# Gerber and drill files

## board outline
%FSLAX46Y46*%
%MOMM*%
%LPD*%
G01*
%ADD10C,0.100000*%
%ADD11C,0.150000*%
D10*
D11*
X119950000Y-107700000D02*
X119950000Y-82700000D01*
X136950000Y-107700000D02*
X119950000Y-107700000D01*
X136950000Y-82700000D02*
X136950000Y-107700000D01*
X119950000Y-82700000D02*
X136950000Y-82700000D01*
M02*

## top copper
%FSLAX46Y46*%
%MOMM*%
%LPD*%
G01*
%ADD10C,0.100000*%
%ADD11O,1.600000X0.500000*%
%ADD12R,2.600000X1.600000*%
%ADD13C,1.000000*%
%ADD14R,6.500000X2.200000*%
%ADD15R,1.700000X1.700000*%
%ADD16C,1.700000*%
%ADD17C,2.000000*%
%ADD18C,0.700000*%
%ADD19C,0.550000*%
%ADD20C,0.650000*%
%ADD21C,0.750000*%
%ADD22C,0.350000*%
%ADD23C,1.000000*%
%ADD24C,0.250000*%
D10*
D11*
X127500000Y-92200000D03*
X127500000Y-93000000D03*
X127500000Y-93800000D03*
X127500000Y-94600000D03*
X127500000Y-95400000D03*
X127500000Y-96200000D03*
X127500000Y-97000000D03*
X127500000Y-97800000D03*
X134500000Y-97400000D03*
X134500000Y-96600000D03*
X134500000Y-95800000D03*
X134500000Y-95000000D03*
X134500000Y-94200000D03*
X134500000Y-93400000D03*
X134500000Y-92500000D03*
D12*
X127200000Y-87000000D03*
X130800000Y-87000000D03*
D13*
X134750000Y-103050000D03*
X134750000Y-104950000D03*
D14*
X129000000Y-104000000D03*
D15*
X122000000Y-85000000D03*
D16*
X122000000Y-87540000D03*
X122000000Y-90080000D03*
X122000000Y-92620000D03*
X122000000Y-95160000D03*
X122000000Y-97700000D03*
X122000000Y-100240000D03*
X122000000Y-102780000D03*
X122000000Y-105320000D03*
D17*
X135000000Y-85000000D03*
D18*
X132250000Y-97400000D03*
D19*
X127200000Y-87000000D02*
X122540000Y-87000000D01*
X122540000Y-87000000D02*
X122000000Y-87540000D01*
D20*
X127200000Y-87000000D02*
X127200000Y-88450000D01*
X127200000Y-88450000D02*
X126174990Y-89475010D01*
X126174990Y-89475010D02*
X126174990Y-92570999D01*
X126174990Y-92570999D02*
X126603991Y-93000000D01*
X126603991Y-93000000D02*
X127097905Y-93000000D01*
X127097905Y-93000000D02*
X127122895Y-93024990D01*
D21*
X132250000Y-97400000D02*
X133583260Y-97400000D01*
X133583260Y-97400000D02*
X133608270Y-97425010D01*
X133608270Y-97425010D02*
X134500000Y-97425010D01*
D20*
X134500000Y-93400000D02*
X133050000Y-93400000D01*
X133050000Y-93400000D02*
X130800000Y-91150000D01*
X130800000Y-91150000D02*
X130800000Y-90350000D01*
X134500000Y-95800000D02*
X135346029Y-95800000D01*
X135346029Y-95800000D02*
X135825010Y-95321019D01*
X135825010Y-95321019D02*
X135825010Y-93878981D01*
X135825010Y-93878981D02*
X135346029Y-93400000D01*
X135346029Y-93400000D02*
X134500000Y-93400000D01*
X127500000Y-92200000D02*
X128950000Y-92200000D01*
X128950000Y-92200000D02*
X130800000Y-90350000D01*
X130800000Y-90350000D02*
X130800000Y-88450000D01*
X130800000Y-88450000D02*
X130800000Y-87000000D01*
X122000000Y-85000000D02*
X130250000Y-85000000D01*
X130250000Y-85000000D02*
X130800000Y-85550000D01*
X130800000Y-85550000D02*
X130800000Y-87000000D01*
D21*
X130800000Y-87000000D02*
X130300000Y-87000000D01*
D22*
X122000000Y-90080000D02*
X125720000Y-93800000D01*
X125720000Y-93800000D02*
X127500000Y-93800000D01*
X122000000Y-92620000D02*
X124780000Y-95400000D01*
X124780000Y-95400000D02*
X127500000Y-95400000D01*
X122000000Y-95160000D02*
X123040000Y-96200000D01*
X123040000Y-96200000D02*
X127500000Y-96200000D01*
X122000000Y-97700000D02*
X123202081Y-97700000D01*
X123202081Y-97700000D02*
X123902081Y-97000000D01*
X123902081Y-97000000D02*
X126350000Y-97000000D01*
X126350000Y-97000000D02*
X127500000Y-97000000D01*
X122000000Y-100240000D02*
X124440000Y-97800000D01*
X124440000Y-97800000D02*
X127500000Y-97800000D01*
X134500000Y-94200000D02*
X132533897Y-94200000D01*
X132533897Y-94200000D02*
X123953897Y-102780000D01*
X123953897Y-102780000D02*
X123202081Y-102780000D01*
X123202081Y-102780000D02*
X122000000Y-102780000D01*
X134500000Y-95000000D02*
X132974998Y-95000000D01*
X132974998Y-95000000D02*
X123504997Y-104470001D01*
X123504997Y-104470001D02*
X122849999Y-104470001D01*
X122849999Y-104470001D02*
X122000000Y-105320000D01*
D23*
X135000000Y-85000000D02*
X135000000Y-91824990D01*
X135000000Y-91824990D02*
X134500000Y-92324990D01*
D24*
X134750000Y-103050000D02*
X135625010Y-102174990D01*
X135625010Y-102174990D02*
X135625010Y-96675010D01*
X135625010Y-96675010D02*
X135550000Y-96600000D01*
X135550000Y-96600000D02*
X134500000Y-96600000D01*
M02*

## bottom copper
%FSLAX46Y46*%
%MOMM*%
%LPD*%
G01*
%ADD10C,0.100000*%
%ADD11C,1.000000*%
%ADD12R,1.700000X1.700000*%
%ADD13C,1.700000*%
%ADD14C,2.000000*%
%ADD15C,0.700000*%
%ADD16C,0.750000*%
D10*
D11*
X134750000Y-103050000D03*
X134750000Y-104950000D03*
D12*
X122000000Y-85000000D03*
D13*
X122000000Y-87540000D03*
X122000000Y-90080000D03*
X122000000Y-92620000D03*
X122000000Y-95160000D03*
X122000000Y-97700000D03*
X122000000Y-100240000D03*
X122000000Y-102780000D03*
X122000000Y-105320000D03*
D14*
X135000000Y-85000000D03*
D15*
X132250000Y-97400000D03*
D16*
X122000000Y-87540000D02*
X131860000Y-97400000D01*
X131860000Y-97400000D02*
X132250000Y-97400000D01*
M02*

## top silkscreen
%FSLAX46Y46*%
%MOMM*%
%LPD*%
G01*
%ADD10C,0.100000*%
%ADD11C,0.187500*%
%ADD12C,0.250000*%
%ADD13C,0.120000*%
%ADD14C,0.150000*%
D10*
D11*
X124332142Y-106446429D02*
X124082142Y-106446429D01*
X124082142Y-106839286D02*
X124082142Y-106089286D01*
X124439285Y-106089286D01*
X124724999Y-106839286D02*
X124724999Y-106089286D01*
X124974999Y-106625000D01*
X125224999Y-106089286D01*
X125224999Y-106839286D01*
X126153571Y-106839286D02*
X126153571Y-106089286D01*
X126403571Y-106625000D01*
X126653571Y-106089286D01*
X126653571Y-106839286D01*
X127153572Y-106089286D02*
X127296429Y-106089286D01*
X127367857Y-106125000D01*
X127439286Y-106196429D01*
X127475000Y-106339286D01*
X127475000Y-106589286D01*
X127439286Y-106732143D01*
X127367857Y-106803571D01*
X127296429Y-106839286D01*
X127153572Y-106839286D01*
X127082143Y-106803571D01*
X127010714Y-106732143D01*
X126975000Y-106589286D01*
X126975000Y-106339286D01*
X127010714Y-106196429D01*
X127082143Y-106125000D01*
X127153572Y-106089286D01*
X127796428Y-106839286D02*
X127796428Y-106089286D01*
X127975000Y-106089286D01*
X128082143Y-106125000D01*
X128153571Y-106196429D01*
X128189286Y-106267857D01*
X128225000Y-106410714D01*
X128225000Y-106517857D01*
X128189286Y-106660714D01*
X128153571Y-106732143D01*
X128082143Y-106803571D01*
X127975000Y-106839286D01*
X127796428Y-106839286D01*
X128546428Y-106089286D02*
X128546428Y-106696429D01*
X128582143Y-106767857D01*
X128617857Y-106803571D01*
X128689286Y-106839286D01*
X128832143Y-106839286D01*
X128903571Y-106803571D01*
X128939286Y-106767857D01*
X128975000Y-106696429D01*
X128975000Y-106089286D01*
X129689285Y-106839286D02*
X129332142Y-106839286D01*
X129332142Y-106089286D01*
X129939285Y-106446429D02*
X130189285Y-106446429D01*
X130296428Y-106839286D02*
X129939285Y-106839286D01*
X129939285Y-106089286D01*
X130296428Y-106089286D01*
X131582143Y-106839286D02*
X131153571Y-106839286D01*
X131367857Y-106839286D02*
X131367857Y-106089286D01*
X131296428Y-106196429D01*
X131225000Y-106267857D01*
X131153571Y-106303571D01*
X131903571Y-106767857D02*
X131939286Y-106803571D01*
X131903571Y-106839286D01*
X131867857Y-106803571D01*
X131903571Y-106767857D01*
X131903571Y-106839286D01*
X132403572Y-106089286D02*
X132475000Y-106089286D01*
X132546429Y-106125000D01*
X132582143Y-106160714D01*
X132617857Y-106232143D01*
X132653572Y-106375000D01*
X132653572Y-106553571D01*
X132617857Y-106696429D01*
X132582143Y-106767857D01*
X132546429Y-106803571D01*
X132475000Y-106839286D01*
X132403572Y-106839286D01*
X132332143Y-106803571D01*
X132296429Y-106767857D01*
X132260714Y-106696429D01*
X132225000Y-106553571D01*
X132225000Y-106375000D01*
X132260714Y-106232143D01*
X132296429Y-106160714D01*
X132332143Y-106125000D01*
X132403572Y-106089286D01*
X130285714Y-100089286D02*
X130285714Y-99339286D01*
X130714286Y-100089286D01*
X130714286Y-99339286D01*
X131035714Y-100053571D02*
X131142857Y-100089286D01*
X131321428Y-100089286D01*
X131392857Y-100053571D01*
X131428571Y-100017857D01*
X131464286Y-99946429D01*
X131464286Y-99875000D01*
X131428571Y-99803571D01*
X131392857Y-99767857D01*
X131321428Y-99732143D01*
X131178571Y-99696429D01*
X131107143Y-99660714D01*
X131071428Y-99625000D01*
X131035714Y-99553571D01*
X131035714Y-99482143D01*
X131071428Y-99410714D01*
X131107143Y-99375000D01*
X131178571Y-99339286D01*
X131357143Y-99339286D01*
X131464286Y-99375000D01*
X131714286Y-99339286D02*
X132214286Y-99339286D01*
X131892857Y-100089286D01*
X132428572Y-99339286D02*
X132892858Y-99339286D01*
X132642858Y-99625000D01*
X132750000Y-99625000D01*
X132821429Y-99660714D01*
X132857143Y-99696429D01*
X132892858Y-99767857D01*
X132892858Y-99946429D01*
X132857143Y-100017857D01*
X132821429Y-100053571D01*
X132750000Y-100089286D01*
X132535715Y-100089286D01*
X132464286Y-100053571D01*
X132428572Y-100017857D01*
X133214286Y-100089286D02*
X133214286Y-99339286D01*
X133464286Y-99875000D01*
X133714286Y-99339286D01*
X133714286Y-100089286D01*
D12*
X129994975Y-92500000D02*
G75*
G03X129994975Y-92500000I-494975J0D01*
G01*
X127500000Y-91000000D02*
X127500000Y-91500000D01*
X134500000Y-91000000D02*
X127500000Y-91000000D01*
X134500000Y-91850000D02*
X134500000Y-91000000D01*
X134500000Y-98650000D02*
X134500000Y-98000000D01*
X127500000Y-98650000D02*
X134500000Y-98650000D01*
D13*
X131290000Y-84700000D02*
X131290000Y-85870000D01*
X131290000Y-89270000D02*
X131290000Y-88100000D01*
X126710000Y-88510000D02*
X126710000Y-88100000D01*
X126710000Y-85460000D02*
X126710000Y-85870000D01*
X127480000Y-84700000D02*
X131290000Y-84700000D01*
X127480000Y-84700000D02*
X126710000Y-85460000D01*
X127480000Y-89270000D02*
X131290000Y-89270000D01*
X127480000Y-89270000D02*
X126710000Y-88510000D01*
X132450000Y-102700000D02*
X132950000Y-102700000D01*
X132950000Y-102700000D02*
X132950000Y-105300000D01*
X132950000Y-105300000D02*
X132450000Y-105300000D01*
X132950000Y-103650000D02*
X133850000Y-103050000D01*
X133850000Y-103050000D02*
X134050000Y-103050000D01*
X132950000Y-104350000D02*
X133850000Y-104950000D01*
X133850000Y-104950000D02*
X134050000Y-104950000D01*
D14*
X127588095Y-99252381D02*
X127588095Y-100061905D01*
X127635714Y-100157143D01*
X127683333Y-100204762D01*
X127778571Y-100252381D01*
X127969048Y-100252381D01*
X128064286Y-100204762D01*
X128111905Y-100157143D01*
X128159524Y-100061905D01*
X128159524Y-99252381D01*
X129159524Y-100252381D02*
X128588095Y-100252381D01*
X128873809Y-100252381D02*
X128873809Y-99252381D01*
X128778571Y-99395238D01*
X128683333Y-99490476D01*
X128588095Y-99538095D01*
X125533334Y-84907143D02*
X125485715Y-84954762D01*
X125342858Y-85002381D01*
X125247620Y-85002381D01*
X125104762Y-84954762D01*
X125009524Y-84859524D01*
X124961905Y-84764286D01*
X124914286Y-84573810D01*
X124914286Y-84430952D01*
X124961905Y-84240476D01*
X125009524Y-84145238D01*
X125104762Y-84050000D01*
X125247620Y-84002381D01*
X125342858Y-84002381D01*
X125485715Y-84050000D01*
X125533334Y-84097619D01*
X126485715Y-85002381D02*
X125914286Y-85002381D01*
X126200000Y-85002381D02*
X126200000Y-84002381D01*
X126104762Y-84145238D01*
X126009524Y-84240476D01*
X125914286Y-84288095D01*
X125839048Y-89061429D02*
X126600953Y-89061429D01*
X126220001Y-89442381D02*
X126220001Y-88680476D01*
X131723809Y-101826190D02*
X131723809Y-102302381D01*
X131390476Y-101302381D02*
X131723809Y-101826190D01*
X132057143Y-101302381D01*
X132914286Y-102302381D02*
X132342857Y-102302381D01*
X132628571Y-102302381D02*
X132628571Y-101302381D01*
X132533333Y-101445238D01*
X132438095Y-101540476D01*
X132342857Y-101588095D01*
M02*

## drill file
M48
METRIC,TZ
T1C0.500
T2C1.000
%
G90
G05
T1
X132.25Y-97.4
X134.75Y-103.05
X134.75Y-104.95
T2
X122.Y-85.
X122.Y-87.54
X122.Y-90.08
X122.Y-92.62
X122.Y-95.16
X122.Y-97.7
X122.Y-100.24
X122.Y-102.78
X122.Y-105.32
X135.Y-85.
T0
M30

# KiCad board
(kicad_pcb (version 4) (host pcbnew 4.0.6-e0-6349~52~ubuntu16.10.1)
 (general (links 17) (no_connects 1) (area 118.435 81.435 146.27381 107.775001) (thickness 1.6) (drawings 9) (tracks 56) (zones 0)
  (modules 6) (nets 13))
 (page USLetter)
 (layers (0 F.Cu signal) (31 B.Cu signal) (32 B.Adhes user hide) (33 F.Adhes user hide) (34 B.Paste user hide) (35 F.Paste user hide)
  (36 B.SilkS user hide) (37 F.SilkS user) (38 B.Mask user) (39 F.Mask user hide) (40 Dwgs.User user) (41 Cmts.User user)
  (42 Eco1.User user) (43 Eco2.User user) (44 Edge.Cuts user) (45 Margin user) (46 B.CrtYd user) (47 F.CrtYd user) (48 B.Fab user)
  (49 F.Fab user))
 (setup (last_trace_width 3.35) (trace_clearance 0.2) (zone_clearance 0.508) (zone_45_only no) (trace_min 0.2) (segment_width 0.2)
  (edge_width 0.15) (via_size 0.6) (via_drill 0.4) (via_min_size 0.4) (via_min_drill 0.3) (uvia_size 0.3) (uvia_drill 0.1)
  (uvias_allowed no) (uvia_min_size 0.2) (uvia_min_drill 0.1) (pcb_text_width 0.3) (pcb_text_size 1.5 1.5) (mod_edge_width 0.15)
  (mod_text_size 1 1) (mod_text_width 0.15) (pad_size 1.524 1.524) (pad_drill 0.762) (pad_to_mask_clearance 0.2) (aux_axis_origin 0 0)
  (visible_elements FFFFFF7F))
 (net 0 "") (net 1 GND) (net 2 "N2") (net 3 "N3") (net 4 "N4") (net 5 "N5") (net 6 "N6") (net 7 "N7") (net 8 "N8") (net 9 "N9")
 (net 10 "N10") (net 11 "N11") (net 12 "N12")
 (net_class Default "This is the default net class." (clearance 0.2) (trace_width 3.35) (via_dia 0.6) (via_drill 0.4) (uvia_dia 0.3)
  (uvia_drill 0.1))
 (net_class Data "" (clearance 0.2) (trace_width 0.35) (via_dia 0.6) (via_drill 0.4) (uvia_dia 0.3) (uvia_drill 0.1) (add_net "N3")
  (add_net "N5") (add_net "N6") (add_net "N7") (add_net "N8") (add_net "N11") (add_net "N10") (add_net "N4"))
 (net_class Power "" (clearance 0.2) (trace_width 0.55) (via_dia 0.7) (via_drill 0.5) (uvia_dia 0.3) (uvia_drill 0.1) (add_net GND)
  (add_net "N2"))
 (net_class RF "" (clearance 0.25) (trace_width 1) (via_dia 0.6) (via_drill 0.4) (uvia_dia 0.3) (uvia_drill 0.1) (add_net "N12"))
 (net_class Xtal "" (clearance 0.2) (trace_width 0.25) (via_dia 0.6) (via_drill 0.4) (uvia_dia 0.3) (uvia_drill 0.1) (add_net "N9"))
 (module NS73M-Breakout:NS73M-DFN (layer F.Cu) (at 131 95 180)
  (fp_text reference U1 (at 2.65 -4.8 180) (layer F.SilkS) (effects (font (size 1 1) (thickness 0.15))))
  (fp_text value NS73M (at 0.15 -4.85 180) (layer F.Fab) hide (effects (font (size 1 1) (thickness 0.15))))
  (fp_circle (center 1.5 2.5) (end 1.15 2.15) (layer F.SilkS) (width 0.25))
  (fp_line (start 3.5 4) (end 3.5 3.5) (layer F.SilkS) (width 0.25))
  (fp_line (start -3.5 4) (end 3.5 4) (layer F.SilkS) (width 0.25))
  (fp_line (start -3.5 3.15) (end -3.5 4) (layer F.SilkS) (width 0.25))
  (fp_line (start -3.5 -3.65) (end -3.5 -3) (layer F.SilkS) (width 0.25))
  (fp_line (start 3.5 -3.65) (end -3.5 -3.65) (layer F.SilkS) (width 0.25))
  (pad 1 smd oval (at 3.5 2.8 180) (size 1.6 0.5) (layers F.Cu F.Paste F.Mask) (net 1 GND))
  (pad 2 smd oval (at 3.5 2 180) (size 1.6 0.5) (layers F.Cu F.Paste F.Mask) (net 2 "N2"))
  (pad 3 smd oval (at 3.5 1.2 180) (size 1.6 0.5) (layers F.Cu F.Paste F.Mask) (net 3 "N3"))
  (pad 4 smd oval (at 3.5 0.4 180) (size 1.6 0.5) (layers F.Cu F.Paste F.Mask) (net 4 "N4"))
  (pad 5 smd oval (at 3.5 -0.4 180) (size 1.6 0.5) (layers F.Cu F.Paste F.Mask) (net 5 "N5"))
  (pad 6 smd oval (at 3.5 -1.2 180) (size 1.6 0.5) (layers F.Cu F.Paste F.Mask) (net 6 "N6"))
  (pad 7 smd oval (at 3.5 -2 180) (size 1.6 0.5) (layers F.Cu F.Paste F.Mask) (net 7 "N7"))
  (pad 8 smd oval (at 3.5 -2.8 180) (size 1.6 0.5) (layers F.Cu F.Paste F.Mask) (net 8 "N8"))
  (pad 9 smd oval (at -3.5 -2.4 180) (size 1.6 0.5) (layers F.Cu F.Paste F.Mask) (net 2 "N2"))
  (pad 10 smd oval (at -3.5 -1.6 180) (size 1.6 0.5) (layers F.Cu F.Paste F.Mask) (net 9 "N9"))
  (pad 11 smd oval (at -3.5 -0.8 180) (size 1.6 0.5) (layers F.Cu F.Paste F.Mask) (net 1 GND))
  (pad 12 smd oval (at -3.5 0 180) (size 1.6 0.5) (layers F.Cu F.Paste F.Mask) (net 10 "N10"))
  (pad 13 smd oval (at -3.5 0.8 180) (size 1.6 0.5) (layers F.Cu F.Paste F.Mask) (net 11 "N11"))
  (pad 14 smd oval (at -3.5 1.6 180) (size 1.6 0.5) (layers F.Cu F.Paste F.Mask) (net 1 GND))
  (pad 15 smd oval (at -3.5 2.5 180) (size 1.6 0.5) (layers F.Cu F.Paste F.Mask) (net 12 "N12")))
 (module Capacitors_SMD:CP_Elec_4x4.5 (layer F.Cu) (at 129 87)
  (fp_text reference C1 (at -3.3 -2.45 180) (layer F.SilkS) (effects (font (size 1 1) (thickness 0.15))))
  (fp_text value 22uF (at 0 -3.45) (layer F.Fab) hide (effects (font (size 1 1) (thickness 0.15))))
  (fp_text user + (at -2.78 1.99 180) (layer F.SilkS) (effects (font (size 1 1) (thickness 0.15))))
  (fp_line (start 2.29 -2.3) (end 2.29 -1.13) (layer F.SilkS) (width 0.12))
  (fp_line (start 2.29 2.27) (end 2.29 1.1) (layer F.SilkS) (width 0.12))
  (fp_line (start -2.29 1.51) (end -2.29 1.1) (layer F.SilkS) (width 0.12))
  (fp_line (start -2.29 -1.54) (end -2.29 -1.13) (layer F.SilkS) (width 0.12))
  (fp_line (start -1.52 -2.3) (end 2.29 -2.3) (layer F.SilkS) (width 0.12))
  (fp_line (start -1.52 -2.3) (end -2.29 -1.54) (layer F.SilkS) (width 0.12))
  (fp_line (start -1.52 2.27) (end 2.29 2.27) (layer F.SilkS) (width 0.12))
  (fp_line (start -1.52 2.27) (end -2.29 1.51) (layer F.SilkS) (width 0.12))
  (pad 1 smd rect (at -1.8 0 180) (size 2.6 1.6) (layers F.Cu F.Paste F.Mask) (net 2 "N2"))
  (pad 2 smd rect (at 1.8 0 180) (size 2.6 1.6) (layers F.Cu F.Paste F.Mask) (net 1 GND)))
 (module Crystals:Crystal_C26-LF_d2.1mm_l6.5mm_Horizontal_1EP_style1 (layer F.Cu) (at 134.75 103.05 270)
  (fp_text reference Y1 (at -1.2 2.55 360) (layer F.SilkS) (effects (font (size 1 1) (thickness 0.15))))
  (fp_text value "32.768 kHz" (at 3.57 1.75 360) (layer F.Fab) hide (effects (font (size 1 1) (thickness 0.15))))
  (fp_line (start -0.35 2.3) (end -0.35 1.8) (layer F.SilkS) (width 0.12))
  (fp_line (start -0.35 1.8) (end 2.25 1.8) (layer F.SilkS) (width 0.12))
  (fp_line (start 2.25 1.8) (end 2.25 2.3) (layer F.SilkS) (width 0.12))
  (fp_line (start 0.6 1.8) (end 0 0.9) (layer F.SilkS) (width 0.12))
  (fp_line (start 0 0.9) (end 0 0.7) (layer F.SilkS) (width 0.12))
  (fp_line (start 1.3 1.8) (end 1.9 0.9) (layer F.SilkS) (width 0.12))
  (fp_line (start 1.9 0.9) (end 1.9 0.7) (layer F.SilkS) (width 0.12))
  (pad 1 thru_hole circle (at 0 0 270) (size 1 1) (drill 0.5) (layers *.Cu *.Mask) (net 9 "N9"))
  (pad 2 thru_hole circle (at 1.9 0 270) (size 1 1) (drill 0.5) (layers *.Cu *.Mask) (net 1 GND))
  (pad 3 smd rect (at 0.95 5.75 270) (size 2.2 6.5) (layers F.Cu F.Paste F.Mask)))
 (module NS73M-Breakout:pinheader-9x (layer F.Cu) (at 122 85)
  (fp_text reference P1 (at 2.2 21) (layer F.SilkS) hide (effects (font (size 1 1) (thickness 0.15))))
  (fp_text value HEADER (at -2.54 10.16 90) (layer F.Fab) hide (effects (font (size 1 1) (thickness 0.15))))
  (pad 1 thru_hole rect (at 0 0) (size 1.7 1.7) (drill 1) (layers *.Cu *.Mask) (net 1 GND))
  (pad 2 thru_hole circle (at 0 2.54) (size 1.7 1.7) (drill 1) (layers *.Cu *.Mask) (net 2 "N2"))
  (pad 3 thru_hole circle (at 0 5.08) (size 1.7 1.7) (drill 1) (layers *.Cu *.Mask) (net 3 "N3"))
  (pad 4 thru_hole circle (at 0 7.62) (size 1.7 1.7) (drill 1) (layers *.Cu *.Mask) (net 5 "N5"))
  (pad 5 thru_hole circle (at 0 10.16) (size 1.7 1.7) (drill 1) (layers *.Cu *.Mask) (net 6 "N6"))
  (pad 6 thru_hole circle (at 0 12.7) (size 1.7 1.7) (drill 1) (layers *.Cu *.Mask) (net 7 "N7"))
  (pad 7 thru_hole circle (at 0 15.24) (size 1.7 1.7) (drill 1) (layers *.Cu *.Mask) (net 8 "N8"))
  (pad 8 thru_hole circle (at 0 17.78) (size 1.7 1.7) (drill 1) (layers *.Cu *.Mask) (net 11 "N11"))
  (pad 9 thru_hole circle (at 0 20.32) (size 1.7 1.7) (drill 1) (layers *.Cu *.Mask) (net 10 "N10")))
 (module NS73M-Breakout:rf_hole (layer F.Cu) (at 135 85)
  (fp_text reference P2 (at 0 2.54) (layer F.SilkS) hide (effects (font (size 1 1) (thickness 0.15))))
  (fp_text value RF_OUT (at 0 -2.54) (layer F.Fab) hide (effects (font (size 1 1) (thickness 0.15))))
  (pad 1 thru_hole circle (at 0 0) (size 2 2) (drill 1) (layers *.Cu *.Mask) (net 12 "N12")))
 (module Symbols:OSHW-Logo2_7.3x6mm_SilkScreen (layer B.Cu) (at 132.25 96.95)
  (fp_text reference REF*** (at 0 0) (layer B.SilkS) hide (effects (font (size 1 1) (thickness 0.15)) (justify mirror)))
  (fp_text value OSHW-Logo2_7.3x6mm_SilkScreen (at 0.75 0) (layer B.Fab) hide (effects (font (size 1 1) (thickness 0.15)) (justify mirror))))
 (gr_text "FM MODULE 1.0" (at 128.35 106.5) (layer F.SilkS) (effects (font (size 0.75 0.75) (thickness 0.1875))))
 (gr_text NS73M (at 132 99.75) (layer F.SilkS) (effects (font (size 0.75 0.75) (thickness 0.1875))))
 (gr_line (start 119.95 107.7) (end 119.95 82.7) (layer Edge.Cuts) (width 0.15))
 (gr_line (start 136.95 107.7) (end 119.95 107.7) (layer Edge.Cuts) (width 0.15))
 (gr_line (start 136.95 82.7) (end 136.95 107.7) (layer Edge.Cuts) (width 0.15))
 (gr_line (start 119.95 82.7) (end 136.95 82.7) (layer Edge.Cuts) (width 0.15))
 (segment (start 127.2 87) (end 122.54 87) (width 0.55) (layer F.Cu) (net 2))
 (segment (start 122.54 87) (end 122 87.54) (width 0.55) (layer F.Cu) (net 2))
 (segment (start 127.2 87) (end 127.2 88.45) (width 0.65) (layer F.Cu) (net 2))
 (segment (start 127.2 88.45) (end 126.17499 89.47501) (width 0.65) (layer F.Cu) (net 2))
 (segment (start 126.17499 89.47501) (end 126.17499 92.570999) (width 0.65) (layer F.Cu) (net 2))
 (segment (start 126.17499 92.570999) (end 126.603991 93) (width 0.65) (layer F.Cu) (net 2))
 (segment (start 126.603991 93) (end 127.097905 93) (width 0.65) (layer F.Cu) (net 2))
 (segment (start 127.097905 93) (end 127.122895 93.02499) (width 0.65) (layer F.Cu) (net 2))
 (segment (start 132.25 97.4) (end 133.58326 97.4) (width 0.75) (layer F.Cu) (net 2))
 (segment (start 133.58326 97.4) (end 133.60827 97.42501) (width 0.75) (layer F.Cu) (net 2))
 (segment (start 133.60827 97.42501) (end 134.5 97.42501) (width 0.75) (layer F.Cu) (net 2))
 (segment (start 122 87.54) (end 131.86 97.4) (width 0.75) (layer B.Cu) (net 2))
 (segment (start 131.86 97.4) (end 132.25 97.4) (width 0.75) (layer B.Cu) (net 2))
 (via (at 132.25 97.4) (size 0.7) (drill 0.5) (layers F.Cu B.Cu) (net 2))
 (segment (start 134.5 93.4) (end 133.05 93.4) (width 0.65) (layer F.Cu) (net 1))
 (segment (start 133.05 93.4) (end 130.8 91.15) (width 0.65) (layer F.Cu) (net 1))
 (segment (start 130.8 91.15) (end 130.8 90.35) (width 0.65) (layer F.Cu) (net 1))
 (segment (start 134.5 95.8) (end 135.346029 95.8) (width 0.65) (layer F.Cu) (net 1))
 (segment (start 135.346029 95.8) (end 135.82501 95.321019) (width 0.65) (layer F.Cu) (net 1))
 (segment (start 135.82501 95.321019) (end 135.82501 93.878981) (width 0.65) (layer F.Cu) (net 1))
 (segment (start 135.82501 93.878981) (end 135.346029 93.4) (width 0.65) (layer F.Cu) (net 1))
 (segment (start 135.346029 93.4) (end 134.5 93.4) (width 0.65) (layer F.Cu) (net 1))
 (segment (start 127.5 92.2) (end 128.95 92.2) (width 0.65) (layer F.Cu) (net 1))
 (segment (start 128.95 92.2) (end 130.8 90.35) (width 0.65) (layer F.Cu) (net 1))
 (segment (start 130.8 90.35) (end 130.8 88.45) (width 0.65) (layer F.Cu) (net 1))
 (segment (start 130.8 88.45) (end 130.8 87) (width 0.65) (layer F.Cu) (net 1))
 (segment (start 122 85) (end 130.25 85) (width 0.65) (layer F.Cu) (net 1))
 (segment (start 130.25 85) (end 130.8 85.55) (width 0.65) (layer F.Cu) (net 1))
 (segment (start 130.8 85.55) (end 130.8 87) (width 0.65) (layer F.Cu) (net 1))
 (segment (start 130.8 87) (end 130.3 87) (width 0.75) (layer F.Cu) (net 1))
 (segment (start 122 90.08) (end 125.72 93.8) (width 0.35) (layer F.Cu) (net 3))
 (segment (start 125.72 93.8) (end 127.5 93.8) (width 0.35) (layer F.Cu) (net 3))
 (segment (start 122 92.62) (end 124.78 95.4) (width 0.35) (layer F.Cu) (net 5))
 (segment (start 124.78 95.4) (end 127.5 95.4) (width 0.35) (layer F.Cu) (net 5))
 (segment (start 122 95.16) (end 123.04 96.2) (width 0.35) (layer F.Cu) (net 6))
 (segment (start 123.04 96.2) (end 127.5 96.2) (width 0.35) (layer F.Cu) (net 6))
 (segment (start 122 97.7) (end 123.202081 97.7) (width 0.35) (layer F.Cu) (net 7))
 (segment (start 123.202081 97.7) (end 123.902081 97) (width 0.35) (layer F.Cu) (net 7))
 (segment (start 123.902081 97) (end 126.35 97) (width 0.35) (layer F.Cu) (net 7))
 (segment (start 126.35 97) (end 127.5 97) (width 0.35) (layer F.Cu) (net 7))
 (segment (start 122 100.24) (end 124.44 97.8) (width 0.35) (layer F.Cu) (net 8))
 (segment (start 124.44 97.8) (end 127.5 97.8) (width 0.35) (layer F.Cu) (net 8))
 (segment (start 134.5 94.2) (end 132.533897 94.2) (width 0.35) (layer F.Cu) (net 11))
 (segment (start 132.533897 94.2) (end 123.953897 102.78) (width 0.35) (layer F.Cu) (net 11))
 (segment (start 123.953897 102.78) (end 123.202081 102.78) (width 0.35) (layer F.Cu) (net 11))
 (segment (start 123.202081 102.78) (end 122 102.78) (width 0.35) (layer F.Cu) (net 11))
 (segment (start 134.5 95) (end 132.974998 95) (width 0.35) (layer F.Cu) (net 10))
 (segment (start 132.974998 95) (end 123.504997 104.470001) (width 0.35) (layer F.Cu) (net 10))
 (segment (start 123.504997 104.470001) (end 122.849999 104.470001) (width 0.35) (layer F.Cu) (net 10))
 (segment (start 122.849999 104.470001) (end 122 105.32) (width 0.35) (layer F.Cu) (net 10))
 (segment (start 135 85) (end 135 91.82499) (width 1) (layer F.Cu) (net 12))
 (segment (start 135 91.82499) (end 134.5 92.32499) (width 1) (layer F.Cu) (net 12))
 (segment (start 134.75 103.05) (end 135.62501 102.17499) (width 0.25) (layer F.Cu) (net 9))
 (segment (start 135.62501 102.17499) (end 135.62501 96.67501) (width 0.25) (layer F.Cu) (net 9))
 (segment (start 135.62501 96.67501) (end 135.55 96.6) (width 0.25) (layer F.Cu) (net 9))
 (segment (start 135.55 96.6) (end 134.5 96.6) (width 0.25) (layer F.Cu) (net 9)))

